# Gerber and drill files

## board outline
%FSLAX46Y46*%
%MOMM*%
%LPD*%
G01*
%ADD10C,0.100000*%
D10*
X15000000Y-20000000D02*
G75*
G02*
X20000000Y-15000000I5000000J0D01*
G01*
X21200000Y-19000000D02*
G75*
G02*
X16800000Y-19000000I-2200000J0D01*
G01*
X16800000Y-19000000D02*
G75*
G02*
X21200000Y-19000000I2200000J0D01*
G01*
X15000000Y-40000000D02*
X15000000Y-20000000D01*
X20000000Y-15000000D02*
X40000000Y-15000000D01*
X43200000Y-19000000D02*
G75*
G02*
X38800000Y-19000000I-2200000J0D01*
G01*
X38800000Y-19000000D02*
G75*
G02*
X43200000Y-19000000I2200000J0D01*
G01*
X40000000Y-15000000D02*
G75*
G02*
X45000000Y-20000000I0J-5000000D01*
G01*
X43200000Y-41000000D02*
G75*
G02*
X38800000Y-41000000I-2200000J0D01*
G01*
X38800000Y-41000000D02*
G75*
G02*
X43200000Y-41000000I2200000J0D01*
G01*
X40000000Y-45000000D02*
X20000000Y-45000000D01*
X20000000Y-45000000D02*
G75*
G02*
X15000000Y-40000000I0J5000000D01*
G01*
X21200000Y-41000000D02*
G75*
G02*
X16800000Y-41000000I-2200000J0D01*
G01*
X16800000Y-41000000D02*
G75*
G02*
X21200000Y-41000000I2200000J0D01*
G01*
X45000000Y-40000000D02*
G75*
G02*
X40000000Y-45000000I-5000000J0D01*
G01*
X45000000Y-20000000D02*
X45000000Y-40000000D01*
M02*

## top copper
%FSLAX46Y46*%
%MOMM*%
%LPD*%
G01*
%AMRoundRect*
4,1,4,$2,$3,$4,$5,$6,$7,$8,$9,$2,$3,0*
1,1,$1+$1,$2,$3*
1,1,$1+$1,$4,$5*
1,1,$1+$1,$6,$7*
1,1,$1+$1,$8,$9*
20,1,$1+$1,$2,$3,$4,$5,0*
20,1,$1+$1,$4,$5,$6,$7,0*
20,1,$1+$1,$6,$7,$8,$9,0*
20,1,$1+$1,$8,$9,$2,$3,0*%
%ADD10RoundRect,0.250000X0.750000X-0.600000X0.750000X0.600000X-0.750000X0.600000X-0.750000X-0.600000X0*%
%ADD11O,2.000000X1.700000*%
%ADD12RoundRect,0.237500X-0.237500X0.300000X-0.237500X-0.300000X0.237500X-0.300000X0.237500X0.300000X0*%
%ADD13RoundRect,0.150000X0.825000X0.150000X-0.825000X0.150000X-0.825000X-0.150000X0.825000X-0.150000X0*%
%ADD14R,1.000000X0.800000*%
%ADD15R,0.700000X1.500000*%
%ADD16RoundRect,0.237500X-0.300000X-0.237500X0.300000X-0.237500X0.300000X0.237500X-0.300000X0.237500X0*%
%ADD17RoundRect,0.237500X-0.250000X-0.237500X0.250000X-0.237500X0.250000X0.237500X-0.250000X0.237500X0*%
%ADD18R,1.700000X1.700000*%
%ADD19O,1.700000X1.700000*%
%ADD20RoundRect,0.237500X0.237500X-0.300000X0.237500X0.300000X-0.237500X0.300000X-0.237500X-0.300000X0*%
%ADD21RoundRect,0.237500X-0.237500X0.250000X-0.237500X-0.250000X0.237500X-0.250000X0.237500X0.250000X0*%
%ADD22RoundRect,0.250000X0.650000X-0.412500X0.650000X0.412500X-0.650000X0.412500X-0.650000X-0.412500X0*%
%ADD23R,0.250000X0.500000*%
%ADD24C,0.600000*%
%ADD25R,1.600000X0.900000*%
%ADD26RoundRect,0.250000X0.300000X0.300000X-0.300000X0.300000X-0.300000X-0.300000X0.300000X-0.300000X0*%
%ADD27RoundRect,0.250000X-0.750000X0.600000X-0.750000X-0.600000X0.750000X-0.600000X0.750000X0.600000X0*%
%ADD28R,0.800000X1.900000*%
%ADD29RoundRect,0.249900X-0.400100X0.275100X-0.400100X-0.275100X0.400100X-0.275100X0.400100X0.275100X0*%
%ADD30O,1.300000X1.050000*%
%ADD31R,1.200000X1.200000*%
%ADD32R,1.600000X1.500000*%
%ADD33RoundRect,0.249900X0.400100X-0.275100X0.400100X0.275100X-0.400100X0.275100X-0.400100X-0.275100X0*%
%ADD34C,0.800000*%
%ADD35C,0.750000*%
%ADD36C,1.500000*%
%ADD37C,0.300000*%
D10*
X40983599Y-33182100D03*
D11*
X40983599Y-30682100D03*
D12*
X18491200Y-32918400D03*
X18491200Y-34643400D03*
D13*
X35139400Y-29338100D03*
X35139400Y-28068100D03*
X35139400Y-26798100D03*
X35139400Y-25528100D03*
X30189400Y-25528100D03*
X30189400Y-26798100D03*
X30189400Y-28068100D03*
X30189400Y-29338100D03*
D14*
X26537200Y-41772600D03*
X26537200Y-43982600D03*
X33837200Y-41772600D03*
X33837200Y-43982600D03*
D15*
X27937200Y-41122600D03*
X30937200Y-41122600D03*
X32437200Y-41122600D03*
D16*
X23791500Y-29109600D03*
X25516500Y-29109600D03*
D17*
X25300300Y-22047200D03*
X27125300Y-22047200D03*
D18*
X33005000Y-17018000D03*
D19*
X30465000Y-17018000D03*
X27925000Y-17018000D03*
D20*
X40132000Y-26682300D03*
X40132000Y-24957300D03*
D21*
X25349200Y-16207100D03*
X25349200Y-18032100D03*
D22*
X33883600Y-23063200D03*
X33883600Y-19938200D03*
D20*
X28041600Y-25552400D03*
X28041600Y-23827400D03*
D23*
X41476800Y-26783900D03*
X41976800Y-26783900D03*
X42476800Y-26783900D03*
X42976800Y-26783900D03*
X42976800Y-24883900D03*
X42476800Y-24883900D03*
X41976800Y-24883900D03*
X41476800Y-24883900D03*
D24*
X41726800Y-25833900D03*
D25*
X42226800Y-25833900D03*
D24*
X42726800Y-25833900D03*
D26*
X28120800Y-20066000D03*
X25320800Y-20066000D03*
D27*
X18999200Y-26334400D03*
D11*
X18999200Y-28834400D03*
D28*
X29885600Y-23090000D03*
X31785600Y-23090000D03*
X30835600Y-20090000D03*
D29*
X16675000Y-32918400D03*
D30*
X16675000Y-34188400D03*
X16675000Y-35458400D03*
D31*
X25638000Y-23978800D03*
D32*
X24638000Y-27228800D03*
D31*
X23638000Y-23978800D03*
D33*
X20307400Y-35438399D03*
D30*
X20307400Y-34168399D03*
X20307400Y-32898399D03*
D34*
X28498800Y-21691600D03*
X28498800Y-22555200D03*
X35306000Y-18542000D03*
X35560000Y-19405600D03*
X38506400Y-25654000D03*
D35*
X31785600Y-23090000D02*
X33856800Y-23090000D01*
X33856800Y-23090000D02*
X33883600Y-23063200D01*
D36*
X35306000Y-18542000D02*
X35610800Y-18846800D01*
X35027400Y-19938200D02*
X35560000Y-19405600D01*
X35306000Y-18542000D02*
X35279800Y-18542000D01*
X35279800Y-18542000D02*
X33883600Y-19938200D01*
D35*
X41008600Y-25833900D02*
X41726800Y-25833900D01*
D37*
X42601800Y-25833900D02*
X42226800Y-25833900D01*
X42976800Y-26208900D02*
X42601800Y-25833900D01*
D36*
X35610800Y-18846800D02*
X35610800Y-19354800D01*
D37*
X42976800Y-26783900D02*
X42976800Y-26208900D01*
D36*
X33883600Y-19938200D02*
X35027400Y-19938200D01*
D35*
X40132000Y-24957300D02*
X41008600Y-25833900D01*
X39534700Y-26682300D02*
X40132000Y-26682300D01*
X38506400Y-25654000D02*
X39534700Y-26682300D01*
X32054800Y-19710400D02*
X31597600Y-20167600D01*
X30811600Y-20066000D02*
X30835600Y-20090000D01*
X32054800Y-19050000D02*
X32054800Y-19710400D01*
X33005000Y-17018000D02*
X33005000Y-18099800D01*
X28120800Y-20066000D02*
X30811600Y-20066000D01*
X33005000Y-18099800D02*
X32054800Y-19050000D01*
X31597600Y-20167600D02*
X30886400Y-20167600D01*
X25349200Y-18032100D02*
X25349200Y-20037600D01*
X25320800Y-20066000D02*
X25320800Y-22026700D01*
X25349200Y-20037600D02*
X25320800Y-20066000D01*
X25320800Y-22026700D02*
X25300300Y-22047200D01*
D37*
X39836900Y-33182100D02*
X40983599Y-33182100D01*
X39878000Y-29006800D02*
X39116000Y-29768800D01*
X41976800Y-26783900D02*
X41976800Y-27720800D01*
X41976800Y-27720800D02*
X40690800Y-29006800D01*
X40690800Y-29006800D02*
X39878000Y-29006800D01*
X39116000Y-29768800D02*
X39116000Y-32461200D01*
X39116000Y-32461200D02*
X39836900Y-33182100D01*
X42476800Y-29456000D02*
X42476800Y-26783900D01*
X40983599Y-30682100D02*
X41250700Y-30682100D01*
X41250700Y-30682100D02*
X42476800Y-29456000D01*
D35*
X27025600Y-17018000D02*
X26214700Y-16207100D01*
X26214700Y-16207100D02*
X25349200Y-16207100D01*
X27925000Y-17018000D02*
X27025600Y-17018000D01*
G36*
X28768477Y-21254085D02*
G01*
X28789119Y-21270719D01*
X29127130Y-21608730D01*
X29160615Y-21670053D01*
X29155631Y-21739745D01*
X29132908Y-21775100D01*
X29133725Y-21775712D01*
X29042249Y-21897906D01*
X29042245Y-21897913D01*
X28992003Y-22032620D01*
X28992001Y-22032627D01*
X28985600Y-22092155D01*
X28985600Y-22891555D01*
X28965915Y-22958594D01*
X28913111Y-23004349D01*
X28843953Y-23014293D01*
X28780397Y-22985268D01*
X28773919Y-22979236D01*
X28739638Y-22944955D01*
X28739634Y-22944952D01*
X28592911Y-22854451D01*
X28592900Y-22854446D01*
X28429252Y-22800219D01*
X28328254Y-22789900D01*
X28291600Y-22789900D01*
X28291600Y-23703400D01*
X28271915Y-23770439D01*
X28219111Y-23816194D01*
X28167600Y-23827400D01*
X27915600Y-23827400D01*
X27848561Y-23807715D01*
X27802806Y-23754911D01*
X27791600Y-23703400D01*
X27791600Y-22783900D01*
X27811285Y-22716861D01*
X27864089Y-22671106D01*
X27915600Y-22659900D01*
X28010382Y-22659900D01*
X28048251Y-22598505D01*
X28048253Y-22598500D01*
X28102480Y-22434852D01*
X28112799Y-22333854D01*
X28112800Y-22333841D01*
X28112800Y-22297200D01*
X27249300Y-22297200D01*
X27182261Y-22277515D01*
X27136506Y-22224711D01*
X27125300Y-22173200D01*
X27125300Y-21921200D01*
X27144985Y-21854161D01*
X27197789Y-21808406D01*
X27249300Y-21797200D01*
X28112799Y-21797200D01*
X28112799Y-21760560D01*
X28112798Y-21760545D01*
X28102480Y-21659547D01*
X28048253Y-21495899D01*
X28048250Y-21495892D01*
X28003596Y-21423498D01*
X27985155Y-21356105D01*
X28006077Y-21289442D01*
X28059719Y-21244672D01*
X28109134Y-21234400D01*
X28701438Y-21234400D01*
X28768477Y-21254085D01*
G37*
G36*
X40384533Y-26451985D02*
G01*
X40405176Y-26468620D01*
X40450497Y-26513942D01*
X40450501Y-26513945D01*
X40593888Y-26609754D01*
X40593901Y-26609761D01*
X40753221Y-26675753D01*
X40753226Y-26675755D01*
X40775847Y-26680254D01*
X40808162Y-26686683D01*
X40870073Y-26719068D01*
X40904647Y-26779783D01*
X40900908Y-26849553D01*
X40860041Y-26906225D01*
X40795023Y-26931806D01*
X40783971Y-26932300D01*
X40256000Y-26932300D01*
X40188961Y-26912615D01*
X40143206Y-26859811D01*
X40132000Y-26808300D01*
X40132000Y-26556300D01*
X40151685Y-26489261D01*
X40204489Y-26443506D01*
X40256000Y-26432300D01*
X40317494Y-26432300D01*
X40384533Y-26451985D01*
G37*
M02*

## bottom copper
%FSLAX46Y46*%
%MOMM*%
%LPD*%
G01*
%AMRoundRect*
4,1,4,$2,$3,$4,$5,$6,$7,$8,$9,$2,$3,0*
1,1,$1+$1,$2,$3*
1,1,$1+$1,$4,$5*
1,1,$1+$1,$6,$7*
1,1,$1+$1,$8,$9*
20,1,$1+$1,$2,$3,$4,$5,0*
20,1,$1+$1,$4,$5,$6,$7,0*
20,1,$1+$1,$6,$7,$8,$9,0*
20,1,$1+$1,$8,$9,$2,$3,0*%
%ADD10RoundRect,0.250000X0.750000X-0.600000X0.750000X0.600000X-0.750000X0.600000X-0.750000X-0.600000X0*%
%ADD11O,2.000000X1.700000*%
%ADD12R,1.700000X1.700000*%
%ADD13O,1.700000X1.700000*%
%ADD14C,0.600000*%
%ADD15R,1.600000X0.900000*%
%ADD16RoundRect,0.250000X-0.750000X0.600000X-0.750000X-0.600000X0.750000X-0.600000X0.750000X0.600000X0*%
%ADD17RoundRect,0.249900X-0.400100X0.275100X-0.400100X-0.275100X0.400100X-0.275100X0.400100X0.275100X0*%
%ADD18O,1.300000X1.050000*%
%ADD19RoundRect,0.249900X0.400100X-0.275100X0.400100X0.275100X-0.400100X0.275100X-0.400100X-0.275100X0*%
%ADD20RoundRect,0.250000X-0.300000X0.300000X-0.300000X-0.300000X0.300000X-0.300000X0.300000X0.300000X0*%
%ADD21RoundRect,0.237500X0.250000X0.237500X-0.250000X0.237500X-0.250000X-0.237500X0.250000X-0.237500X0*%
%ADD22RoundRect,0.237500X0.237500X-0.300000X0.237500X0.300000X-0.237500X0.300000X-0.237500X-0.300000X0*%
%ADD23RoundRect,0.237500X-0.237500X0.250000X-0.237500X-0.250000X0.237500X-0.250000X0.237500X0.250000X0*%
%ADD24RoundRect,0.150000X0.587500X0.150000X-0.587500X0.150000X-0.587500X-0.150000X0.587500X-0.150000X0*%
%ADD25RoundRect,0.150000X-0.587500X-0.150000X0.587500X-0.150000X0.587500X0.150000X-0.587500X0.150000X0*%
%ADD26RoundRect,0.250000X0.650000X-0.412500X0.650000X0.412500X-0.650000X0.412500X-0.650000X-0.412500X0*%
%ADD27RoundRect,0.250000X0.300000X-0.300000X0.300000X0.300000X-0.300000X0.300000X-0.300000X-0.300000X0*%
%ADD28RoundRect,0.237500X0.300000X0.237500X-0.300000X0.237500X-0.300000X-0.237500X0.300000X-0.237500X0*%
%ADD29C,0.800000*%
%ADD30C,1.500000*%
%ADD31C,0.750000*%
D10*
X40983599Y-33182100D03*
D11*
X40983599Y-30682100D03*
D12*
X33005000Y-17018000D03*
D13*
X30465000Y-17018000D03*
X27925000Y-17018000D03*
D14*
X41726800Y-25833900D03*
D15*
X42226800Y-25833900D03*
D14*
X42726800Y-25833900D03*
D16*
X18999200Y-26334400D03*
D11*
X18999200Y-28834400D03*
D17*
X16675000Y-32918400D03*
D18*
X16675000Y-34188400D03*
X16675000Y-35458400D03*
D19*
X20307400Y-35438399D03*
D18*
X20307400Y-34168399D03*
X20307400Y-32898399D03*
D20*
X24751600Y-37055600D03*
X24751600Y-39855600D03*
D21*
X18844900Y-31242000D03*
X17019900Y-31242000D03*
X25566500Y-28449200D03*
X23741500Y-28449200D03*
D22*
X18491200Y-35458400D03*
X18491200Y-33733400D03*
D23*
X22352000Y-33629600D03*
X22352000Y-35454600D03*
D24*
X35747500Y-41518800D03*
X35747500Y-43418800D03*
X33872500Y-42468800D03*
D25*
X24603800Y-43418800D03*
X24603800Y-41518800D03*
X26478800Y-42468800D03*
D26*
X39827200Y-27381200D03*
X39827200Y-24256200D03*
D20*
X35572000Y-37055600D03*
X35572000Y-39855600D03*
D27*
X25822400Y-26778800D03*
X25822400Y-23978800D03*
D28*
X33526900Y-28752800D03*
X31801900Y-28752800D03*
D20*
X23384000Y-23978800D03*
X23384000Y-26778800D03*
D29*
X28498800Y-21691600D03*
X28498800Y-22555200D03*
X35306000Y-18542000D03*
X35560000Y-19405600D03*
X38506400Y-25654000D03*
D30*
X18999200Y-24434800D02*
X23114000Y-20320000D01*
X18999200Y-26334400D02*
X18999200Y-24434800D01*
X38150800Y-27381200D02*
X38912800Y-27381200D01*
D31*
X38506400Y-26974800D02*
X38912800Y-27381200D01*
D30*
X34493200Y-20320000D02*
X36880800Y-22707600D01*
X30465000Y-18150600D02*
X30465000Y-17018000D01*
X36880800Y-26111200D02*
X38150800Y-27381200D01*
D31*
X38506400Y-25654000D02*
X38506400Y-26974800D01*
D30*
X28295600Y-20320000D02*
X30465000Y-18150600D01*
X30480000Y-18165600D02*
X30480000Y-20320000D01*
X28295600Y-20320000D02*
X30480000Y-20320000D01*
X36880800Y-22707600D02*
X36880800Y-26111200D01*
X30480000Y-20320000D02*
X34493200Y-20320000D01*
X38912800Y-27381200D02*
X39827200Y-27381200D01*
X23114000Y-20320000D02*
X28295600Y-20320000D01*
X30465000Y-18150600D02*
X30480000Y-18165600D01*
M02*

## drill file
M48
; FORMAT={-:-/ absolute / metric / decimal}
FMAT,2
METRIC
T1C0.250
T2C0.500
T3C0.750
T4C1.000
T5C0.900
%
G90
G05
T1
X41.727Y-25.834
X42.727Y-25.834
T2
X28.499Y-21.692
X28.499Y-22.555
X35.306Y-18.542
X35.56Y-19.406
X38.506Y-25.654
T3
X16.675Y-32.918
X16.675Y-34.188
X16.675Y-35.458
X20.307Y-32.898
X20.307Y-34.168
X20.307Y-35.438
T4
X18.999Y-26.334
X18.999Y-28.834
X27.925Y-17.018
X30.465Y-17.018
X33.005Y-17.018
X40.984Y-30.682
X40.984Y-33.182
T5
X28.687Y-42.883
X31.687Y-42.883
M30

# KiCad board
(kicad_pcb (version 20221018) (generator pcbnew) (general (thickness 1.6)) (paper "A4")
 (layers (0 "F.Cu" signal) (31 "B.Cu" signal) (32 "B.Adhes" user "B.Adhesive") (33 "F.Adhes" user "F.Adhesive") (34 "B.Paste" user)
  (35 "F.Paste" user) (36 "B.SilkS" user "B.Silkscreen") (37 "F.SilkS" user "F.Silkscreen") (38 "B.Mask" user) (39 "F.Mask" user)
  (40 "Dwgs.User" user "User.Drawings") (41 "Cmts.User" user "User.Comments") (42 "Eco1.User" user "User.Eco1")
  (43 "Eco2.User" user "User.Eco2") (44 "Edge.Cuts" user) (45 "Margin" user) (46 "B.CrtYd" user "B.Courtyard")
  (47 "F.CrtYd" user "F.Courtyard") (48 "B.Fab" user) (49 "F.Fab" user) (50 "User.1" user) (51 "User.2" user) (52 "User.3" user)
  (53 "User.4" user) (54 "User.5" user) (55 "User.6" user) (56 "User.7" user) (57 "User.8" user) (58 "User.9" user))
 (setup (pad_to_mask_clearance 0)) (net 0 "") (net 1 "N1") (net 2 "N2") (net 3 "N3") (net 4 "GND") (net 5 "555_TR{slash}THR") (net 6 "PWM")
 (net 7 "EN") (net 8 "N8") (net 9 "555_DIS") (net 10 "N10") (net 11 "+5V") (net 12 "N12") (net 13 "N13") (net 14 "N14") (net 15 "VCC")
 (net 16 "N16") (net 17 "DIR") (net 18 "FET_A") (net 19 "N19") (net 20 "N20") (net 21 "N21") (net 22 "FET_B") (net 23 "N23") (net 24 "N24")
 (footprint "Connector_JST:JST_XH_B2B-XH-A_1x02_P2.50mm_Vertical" (layer "F.Cu") (at 40.983599 33.1821 90)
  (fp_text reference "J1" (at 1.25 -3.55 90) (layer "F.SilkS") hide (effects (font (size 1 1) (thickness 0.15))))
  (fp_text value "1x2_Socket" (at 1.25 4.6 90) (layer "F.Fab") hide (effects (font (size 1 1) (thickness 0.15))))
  (pad "1" thru_hole roundrect (at 0 0 90) (size 1.7 2) (drill 1) (layers "*.Cu" "*.Mask") (roundrect_rratio 0.147059) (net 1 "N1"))
  (pad "2" thru_hole oval (at 2.5 0 90) (size 1.7 2) (drill 1) (layers "*.Cu" "*.Mask") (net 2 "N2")))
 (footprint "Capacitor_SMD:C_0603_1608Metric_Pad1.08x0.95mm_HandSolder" (layer "F.Cu") (at 18.4912 33.7809 -90)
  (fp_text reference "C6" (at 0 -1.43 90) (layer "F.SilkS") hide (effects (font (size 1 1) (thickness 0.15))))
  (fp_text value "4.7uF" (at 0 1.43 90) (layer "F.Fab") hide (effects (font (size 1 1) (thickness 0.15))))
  (pad "1" smd roundrect (at -0.8625 0 270) (size 1.075 0.95) (layers "F.Cu" "F.Paste" "F.Mask") (roundrect_rratio 0.25) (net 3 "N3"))
  (pad "2" smd roundrect (at 0.8625 0 270) (size 1.075 0.95) (layers "F.Cu" "F.Paste" "F.Mask") (roundrect_rratio 0.25) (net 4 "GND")))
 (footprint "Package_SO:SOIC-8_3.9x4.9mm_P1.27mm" (layer "F.Cu") (at 32.6644 27.4331 180)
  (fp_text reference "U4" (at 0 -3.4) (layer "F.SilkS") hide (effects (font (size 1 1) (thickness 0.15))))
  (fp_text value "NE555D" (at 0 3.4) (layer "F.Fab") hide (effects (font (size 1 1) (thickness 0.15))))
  (pad "1" smd roundrect (at -2.475 -1.905 180) (size 1.95 0.6) (layers "F.Cu" "F.Paste" "F.Mask") (roundrect_rratio 0.25) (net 4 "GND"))
  (pad "2" smd roundrect (at -2.475 -0.635 180) (size 1.95 0.6) (layers "F.Cu" "F.Paste" "F.Mask") (roundrect_rratio 0.25)
   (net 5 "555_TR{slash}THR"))
  (pad "3" smd roundrect (at -2.475 0.635 180) (size 1.95 0.6) (layers "F.Cu" "F.Paste" "F.Mask") (roundrect_rratio 0.25) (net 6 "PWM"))
  (pad "4" smd roundrect (at -2.475 1.905 180) (size 1.95 0.6) (layers "F.Cu" "F.Paste" "F.Mask") (roundrect_rratio 0.25) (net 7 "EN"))
  (pad "5" smd roundrect (at 2.475 1.905 180) (size 1.95 0.6) (layers "F.Cu" "F.Paste" "F.Mask") (roundrect_rratio 0.25) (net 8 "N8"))
  (pad "6" smd roundrect (at 2.475 0.635 180) (size 1.95 0.6) (layers "F.Cu" "F.Paste" "F.Mask") (roundrect_rratio 0.25)
   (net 5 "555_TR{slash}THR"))
  (pad "7" smd roundrect (at 2.475 -0.635 180) (size 1.95 0.6) (layers "F.Cu" "F.Paste" "F.Mask") (roundrect_rratio 0.25) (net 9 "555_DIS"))
  (pad "8" smd roundrect (at 2.475 -1.905 180) (size 1.95 0.6) (layers "F.Cu" "F.Paste" "F.Mask") (roundrect_rratio 0.25) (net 7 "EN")))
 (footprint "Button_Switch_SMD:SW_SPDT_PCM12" (layer "F.Cu") (at 30.1872 42.5526)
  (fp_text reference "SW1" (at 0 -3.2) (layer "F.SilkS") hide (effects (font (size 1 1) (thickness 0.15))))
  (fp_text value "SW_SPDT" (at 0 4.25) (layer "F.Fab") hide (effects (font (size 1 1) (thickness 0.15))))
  (pad "" smd rect (at -3.65 -0.78) (size 1 0.8) (layers "F.Cu" "F.Paste" "F.Mask"))
  (pad "" smd rect (at -3.65 1.43) (size 1 0.8) (layers "F.Cu" "F.Paste" "F.Mask"))
  (pad "" np_thru_hole circle (at -1.5 0.33) (size 0.9 0.9) (drill 0.9) (layers "*.Cu" "*.Mask"))
  (pad "" np_thru_hole circle (at 1.5 0.33) (size 0.9 0.9) (drill 0.9) (layers "*.Cu" "*.Mask"))
  (pad "" smd rect (at 3.65 -0.78) (size 1 0.8) (layers "F.Cu" "F.Paste" "F.Mask"))
  (pad "" smd rect (at 3.65 1.43) (size 1 0.8) (layers "F.Cu" "F.Paste" "F.Mask"))
  (pad "1" smd rect (at -2.25 -1.43) (size 0.7 1.5) (layers "F.Cu" "F.Paste" "F.Mask") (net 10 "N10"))
  (pad "2" smd rect (at 0.75 -1.43) (size 0.7 1.5) (layers "F.Cu" "F.Paste" "F.Mask") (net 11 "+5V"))
  (pad "3" smd rect (at 2.25 -1.43) (size 0.7 1.5) (layers "F.Cu" "F.Paste" "F.Mask") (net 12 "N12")))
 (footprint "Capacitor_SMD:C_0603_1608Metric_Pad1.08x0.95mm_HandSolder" (layer "F.Cu") (at 24.654 29.1096)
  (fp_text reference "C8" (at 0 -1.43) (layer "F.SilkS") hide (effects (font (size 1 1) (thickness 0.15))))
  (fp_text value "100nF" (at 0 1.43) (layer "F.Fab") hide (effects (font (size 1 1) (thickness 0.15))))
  (pad "1" smd roundrect (at -0.8625 0) (size 1.075 0.95) (layers "F.Cu" "F.Paste" "F.Mask") (roundrect_rratio 0.25)
   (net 5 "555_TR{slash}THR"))
  (pad "2" smd roundrect (at 0.8625 0) (size 1.075 0.95) (layers "F.Cu" "F.Paste" "F.Mask") (roundrect_rratio 0.25) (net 4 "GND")))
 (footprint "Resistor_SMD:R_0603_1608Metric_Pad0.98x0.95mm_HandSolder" (layer "F.Cu") (at 26.2128 22.0472)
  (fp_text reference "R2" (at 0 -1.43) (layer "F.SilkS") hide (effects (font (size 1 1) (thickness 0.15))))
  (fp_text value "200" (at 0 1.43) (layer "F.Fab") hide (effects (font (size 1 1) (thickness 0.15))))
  (pad "1" smd roundrect (at -0.9125 0) (size 0.975 0.95) (layers "F.Cu" "F.Paste" "F.Mask") (roundrect_rratio 0.25) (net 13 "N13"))
  (pad "2" smd roundrect (at 0.9125 0) (size 0.975 0.95) (layers "F.Cu" "F.Paste" "F.Mask") (roundrect_rratio 0.25) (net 4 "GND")))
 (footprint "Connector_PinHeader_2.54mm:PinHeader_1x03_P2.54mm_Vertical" (layer "F.Cu") (at 33.005 17.018 -90)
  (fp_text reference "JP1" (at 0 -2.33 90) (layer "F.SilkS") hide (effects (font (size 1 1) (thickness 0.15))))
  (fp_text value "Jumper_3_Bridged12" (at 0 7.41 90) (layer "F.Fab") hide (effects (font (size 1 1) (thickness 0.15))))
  (pad "1" thru_hole rect (at 0 0 270) (size 1.7 1.7) (drill 1) (layers "*.Cu" "*.Mask") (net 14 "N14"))
  (pad "2" thru_hole oval (at 0 2.54 270) (size 1.7 1.7) (drill 1) (layers "*.Cu" "*.Mask") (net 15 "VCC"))
  (pad "3" thru_hole oval (at 0 5.08 270) (size 1.7 1.7) (drill 1) (layers "*.Cu" "*.Mask") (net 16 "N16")))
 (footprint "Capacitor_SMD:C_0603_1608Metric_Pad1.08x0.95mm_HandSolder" (layer "F.Cu") (at 40.132 25.8198 90)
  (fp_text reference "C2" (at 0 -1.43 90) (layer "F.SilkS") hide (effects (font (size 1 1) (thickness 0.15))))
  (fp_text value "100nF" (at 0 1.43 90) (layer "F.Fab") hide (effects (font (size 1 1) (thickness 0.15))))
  (pad "1" smd roundrect (at -0.8625 0 90) (size 1.075 0.95) (layers "F.Cu" "F.Paste" "F.Mask") (roundrect_rratio 0.25) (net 15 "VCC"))
  (pad "2" smd roundrect (at 0.8625 0 90) (size 1.075 0.95) (layers "F.Cu" "F.Paste" "F.Mask") (roundrect_rratio 0.25) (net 4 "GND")))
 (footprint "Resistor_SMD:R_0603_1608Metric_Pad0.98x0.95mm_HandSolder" (layer "F.Cu") (at 25.3492 17.1196 -90)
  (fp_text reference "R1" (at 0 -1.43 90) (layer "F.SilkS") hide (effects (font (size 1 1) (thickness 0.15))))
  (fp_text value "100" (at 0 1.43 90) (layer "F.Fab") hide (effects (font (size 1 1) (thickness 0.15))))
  (pad "1" smd roundrect (at -0.9125 0 270) (size 0.975 0.95) (layers "F.Cu" "F.Paste" "F.Mask") (roundrect_rratio 0.25) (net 16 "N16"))
  (pad "2" smd roundrect (at 0.9125 0 270) (size 0.975 0.95) (layers "F.Cu" "F.Paste" "F.Mask") (roundrect_rratio 0.25) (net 13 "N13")))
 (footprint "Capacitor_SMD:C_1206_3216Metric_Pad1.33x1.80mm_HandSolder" (layer "F.Cu") (at 33.8836 21.5007 90)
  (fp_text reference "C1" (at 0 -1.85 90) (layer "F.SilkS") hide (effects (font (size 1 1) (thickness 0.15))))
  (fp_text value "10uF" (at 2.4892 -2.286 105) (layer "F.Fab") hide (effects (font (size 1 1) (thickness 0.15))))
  (pad "1" smd roundrect (at -1.5625 0 90) (size 1.325 1.8) (layers "F.Cu" "F.Paste" "F.Mask") (roundrect_rratio 0.188679) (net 11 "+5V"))
  (pad "2" smd roundrect (at 1.5625 0 90) (size 1.325 1.8) (layers "F.Cu" "F.Paste" "F.Mask") (roundrect_rratio 0.188679) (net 4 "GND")))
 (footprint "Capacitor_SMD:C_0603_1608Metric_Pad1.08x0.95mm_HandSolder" (layer "F.Cu") (at 28.0416 24.6899 90)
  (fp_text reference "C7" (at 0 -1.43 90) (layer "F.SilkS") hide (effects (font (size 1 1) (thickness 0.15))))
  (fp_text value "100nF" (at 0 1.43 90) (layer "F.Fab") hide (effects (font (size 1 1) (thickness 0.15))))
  (pad "1" smd roundrect (at -0.8625 0 90) (size 1.075 0.95) (layers "F.Cu" "F.Paste" "F.Mask") (roundrect_rratio 0.25) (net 8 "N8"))
  (pad "2" smd roundrect (at 0.8625 0 90) (size 1.075 0.95) (layers "F.Cu" "F.Paste" "F.Mask") (roundrect_rratio 0.25) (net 4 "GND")))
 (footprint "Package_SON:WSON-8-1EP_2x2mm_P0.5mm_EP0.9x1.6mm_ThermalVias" (layer "F.Cu") (at 42.2268 25.8339 90)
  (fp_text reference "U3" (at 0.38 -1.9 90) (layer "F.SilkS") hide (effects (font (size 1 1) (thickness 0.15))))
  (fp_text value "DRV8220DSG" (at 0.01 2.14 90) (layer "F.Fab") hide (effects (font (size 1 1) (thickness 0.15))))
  (pad "" smd rect (at 0 -0.4 90) (size 0.75 0.65) (layers "F.Paste"))
  (pad "" smd rect (at 0 0.4 90) (size 0.75 0.65) (layers "F.Paste"))
  (pad "1" smd rect (at -0.95 -0.75 90) (size 0.5 0.25) (layers "F.Cu" "F.Paste" "F.Mask") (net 15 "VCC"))
  (pad "2" smd rect (at -0.95 -0.25 90) (size 0.5 0.25) (layers "F.Cu" "F.Paste" "F.Mask") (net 1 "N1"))
  (pad "3" smd rect (at -0.95 0.25 90) (size 0.5 0.25) (layers "F.Cu" "F.Paste" "F.Mask") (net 2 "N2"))
  (pad "4" smd rect (at -0.95 0.75 90) (size 0.5 0.25) (layers "F.Cu" "F.Paste" "F.Mask") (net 4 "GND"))
  (pad "5" smd rect (at 0.95 0.75 90) (size 0.5 0.25) (layers "F.Cu" "F.Paste" "F.Mask") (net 6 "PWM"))
  (pad "6" smd rect (at 0.95 0.25 90) (size 0.5 0.25) (layers "F.Cu" "F.Paste" "F.Mask") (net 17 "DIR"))
  (pad "7" smd rect (at 0.95 -0.25 90) (size 0.5 0.25) (layers "F.Cu" "F.Paste" "F.Mask") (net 11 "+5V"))
  (pad "8" smd rect (at 0.95 -0.75 90) (size 0.5 0.25) (layers "F.Cu" "F.Paste" "F.Mask") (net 7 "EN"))
  (pad "9" thru_hole circle (at 0 -0.5 90) (size 0.6 0.6) (drill 0.25) (layers "*.Cu") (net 4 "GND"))
  (pad "9" smd rect (at 0 0 90) (size 0.9 1.6) (layers "F.Cu" "F.Mask") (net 4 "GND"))
  (pad "9" smd rect (at 0 0 90) (size 0.9 1.6) (layers "B.Cu") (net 4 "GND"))
  (pad "9" thru_hole circle (at 0 0.5 90) (size 0.6 0.6) (drill 0.25) (layers "*.Cu") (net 4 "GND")))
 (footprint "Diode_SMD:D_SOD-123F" (layer "F.Cu") (at 26.7208 20.066 180)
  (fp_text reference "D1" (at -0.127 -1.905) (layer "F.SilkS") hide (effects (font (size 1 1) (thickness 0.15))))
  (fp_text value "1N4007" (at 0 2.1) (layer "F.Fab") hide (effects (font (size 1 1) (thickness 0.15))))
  (pad "1" smd roundrect (at -1.4 0 180) (size 1.1 1.1) (layers "F.Cu" "F.Paste" "F.Mask") (roundrect_rratio 0.2272727273) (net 14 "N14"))
  (pad "2" smd roundrect (at 1.4 0 180) (size 1.1 1.1) (layers "F.Cu" "F.Paste" "F.Mask") (roundrect_rratio 0.2272727273) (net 13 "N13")))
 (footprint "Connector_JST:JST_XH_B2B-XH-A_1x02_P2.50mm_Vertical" (layer "F.Cu") (at 18.9992 26.3344 -90)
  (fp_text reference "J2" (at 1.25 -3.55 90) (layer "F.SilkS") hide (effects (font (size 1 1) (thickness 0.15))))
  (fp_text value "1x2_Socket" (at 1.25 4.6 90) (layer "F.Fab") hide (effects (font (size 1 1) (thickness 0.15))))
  (pad "1" thru_hole roundrect (at 0 0 270) (size 1.7 2) (drill 1) (layers "*.Cu" "*.Mask") (roundrect_rratio 0.147059) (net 15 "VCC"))
  (pad "2" thru_hole oval (at 2.5 0 270) (size 1.7 2) (drill 1) (layers "*.Cu" "*.Mask") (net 4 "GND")))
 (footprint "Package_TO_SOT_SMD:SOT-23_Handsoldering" (layer "F.Cu") (at 30.8356 21.59 90)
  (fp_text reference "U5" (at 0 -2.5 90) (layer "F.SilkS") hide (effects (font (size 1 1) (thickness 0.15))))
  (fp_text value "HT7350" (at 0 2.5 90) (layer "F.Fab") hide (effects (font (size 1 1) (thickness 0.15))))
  (pad "1" smd rect (at -1.5 -0.95 90) (size 1.9 0.8) (layers "F.Cu" "F.Paste" "F.Mask") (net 4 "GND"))
  (pad "2" smd rect (at -1.5 0.95 90) (size 1.9 0.8) (layers "F.Cu" "F.Paste" "F.Mask") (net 11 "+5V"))
  (pad "3" smd rect (at 1.5 0 90) (size 1.9 0.8) (layers "F.Cu" "F.Paste" "F.Mask") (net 14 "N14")))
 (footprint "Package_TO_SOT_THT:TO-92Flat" (layer "F.Cu") (at 16.675 32.9184 -90)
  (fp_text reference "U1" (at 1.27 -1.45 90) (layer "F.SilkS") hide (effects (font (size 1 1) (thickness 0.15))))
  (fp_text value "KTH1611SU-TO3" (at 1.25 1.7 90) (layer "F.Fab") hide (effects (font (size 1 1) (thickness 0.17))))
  (pad "1" thru_hole roundrect (at 0 0 270) (size 1.05 1.3) (drill 0.75) (layers "*.Cu" "*.Mask") (roundrect_rratio 0.238) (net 3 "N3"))
  (pad "2" thru_hole oval (at 1.27 0 270) (size 1.05 1.3) (drill 0.75) (layers "*.Cu" "*.Mask") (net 4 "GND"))
  (pad "3" thru_hole oval (at 2.54 0 270) (size 1.05 1.3) (drill 0.75) (layers "*.Cu" "*.Mask") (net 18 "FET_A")))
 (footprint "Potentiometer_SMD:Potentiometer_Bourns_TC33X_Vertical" (layer "F.Cu") (at 24.638 25.7788 -90)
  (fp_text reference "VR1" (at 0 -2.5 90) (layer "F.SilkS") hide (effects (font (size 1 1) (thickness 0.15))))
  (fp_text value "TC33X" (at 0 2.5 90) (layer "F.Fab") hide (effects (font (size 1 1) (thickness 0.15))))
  (pad "1" smd rect (at -1.8 -1 270) (size 1.2 1.2) (layers "F.Cu" "F.Paste" "F.Mask") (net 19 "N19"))
  (pad "2" smd rect (at 1.45 0 270) (size 1.5 1.6) (layers "F.Cu" "F.Paste" "F.Mask") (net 5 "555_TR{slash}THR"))
  (pad "3" smd rect (at -1.8 1 270) (size 1.2 1.2) (layers "F.Cu" "F.Paste" "F.Mask") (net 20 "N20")))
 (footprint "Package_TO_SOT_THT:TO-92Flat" (layer "F.Cu") (at 20.3074 35.438399 90)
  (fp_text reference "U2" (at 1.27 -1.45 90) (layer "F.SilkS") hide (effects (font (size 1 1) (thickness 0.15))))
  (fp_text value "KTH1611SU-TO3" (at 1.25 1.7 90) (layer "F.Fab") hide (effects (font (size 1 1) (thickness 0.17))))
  (pad "1" thru_hole roundrect (at 0 0 90) (size 1.05 1.3) (drill 0.75) (layers "*.Cu" "*.Mask") (roundrect_rratio 0.238) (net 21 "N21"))
  (pad "2" thru_hole oval (at 1.27 0 90) (size 1.05 1.3) (drill 0.75) (layers "*.Cu" "*.Mask") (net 4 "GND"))
  (pad "3" thru_hole oval (at 2.54 0 90) (size 1.05 1.3) (drill 0.75) (layers "*.Cu" "*.Mask") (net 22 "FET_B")))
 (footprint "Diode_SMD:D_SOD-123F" (layer "B.Cu") (at 24.7516 38.4556 -90)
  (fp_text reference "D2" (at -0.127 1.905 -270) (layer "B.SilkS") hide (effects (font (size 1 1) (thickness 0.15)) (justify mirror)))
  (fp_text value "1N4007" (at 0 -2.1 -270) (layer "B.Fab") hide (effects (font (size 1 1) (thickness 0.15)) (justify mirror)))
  (pad "1" smd roundrect (at -1.4 0 270) (size 1.1 1.1) (layers "B.Cu" "B.Paste" "B.Mask") (roundrect_rratio 0.2272727273) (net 7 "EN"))
  (pad "2" smd roundrect (at 1.4 0 270) (size 1.1 1.1) (layers "B.Cu" "B.Paste" "B.Mask") (roundrect_rratio 0.2272727273) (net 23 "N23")))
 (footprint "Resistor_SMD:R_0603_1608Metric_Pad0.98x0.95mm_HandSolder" (layer "B.Cu") (at 17.9324 31.242 180)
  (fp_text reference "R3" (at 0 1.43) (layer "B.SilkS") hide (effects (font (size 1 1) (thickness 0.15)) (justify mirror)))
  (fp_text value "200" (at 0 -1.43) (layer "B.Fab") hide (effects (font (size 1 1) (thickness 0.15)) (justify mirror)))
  (pad "1" smd roundrect (at -0.9125 0 180) (size 0.975 0.95) (layers "B.Cu" "B.Paste" "B.Mask") (roundrect_rratio 0.25) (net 11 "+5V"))
  (pad "2" smd roundrect (at 0.9125 0 180) (size 0.975 0.95) (layers "B.Cu" "B.Paste" "B.Mask") (roundrect_rratio 0.25) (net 3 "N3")))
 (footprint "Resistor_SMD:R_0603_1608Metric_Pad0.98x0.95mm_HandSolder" (layer "B.Cu") (at 24.654 28.4492 180)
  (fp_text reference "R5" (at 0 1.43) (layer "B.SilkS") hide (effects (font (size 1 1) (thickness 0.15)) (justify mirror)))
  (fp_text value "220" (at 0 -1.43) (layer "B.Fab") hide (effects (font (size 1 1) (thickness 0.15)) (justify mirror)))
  (pad "1" smd roundrect (at -0.9125 0 180) (size 0.975 0.95) (layers "B.Cu" "B.Paste" "B.Mask") (roundrect_rratio 0.25) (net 7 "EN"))
  (pad "2" smd roundrect (at 0.9125 0 180) (size 0.975 0.95) (layers "B.Cu" "B.Paste" "B.Mask") (roundrect_rratio 0.25) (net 9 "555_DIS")))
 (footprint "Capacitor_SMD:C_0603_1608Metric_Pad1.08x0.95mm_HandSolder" (layer "B.Cu") (at 18.4912 34.5959 90)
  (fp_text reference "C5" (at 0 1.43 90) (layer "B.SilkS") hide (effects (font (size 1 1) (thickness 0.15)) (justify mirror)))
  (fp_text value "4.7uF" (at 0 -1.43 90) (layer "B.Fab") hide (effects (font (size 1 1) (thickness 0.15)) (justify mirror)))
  (pad "1" smd roundrect (at -0.8625 0 90) (size 1.075 0.95) (layers "B.Cu" "B.Paste" "B.Mask") (roundrect_rratio 0.25) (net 21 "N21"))
  (pad "2" smd roundrect (at 0.8625 0 90) (size 1.075 0.95) (layers "B.Cu" "B.Paste" "B.Mask") (roundrect_rratio 0.25) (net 4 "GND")))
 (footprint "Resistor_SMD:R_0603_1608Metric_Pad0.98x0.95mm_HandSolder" (layer "B.Cu") (at 22.352 34.5421 -90)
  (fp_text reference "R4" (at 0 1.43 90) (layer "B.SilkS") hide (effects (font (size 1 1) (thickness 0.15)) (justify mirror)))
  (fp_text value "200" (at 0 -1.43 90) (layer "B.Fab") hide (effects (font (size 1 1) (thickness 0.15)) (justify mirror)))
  (pad "1" smd roundrect (at -0.9125 0 270) (size 0.975 0.95) (layers "B.Cu" "B.Paste" "B.Mask") (roundrect_rratio 0.25) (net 11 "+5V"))
  (pad "2" smd roundrect (at 0.9125 0 270) (size 0.975 0.95) (layers "B.Cu" "B.Paste" "B.Mask") (roundrect_rratio 0.25) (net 21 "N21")))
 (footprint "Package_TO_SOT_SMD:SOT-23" (layer "B.Cu") (at 34.81 42.4688 180)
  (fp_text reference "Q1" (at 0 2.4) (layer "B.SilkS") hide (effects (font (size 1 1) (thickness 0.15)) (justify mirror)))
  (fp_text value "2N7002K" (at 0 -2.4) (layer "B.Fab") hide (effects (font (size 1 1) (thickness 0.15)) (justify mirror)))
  (pad "1" smd roundrect (at -0.9375 0.95 180) (size 1.475 0.6) (layers "B.Cu" "B.Paste" "B.Mask") (roundrect_rratio 0.25) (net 18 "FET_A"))
  (pad "2" smd roundrect (at -0.9375 -0.95 180) (size 1.475 0.6) (layers "B.Cu" "B.Paste" "B.Mask") (roundrect_rratio 0.25) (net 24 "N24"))
  (pad "3" smd roundrect (at 0.9375 0 180) (size 1.475 0.6) (layers "B.Cu" "B.Paste" "B.Mask") (roundrect_rratio 0.25) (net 12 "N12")))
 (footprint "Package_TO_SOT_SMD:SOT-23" (layer "B.Cu") (at 25.5413 42.4688)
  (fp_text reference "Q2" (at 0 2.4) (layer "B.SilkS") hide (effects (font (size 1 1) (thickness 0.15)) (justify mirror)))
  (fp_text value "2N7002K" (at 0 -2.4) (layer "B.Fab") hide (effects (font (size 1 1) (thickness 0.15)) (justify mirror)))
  (pad "1" smd roundrect (at -0.9375 0.95) (size 1.475 0.6) (layers "B.Cu" "B.Paste" "B.Mask") (roundrect_rratio 0.25) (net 22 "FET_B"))
  (pad "2" smd roundrect (at -0.9375 -0.95) (size 1.475 0.6) (layers "B.Cu" "B.Paste" "B.Mask") (roundrect_rratio 0.25) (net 23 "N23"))
  (pad "3" smd roundrect (at 0.9375 0) (size 1.475 0.6) (layers "B.Cu" "B.Paste" "B.Mask") (roundrect_rratio 0.25) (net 10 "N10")))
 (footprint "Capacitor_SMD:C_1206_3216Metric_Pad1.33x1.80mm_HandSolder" (layer "B.Cu") (at 39.8272 25.8187 90)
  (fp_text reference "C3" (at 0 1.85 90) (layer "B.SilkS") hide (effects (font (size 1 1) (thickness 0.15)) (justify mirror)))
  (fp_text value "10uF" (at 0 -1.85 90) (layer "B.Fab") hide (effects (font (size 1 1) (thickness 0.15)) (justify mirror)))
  (pad "1" smd roundrect (at -1.5625 0 90) (size 1.325 1.8) (layers "B.Cu" "B.Paste" "B.Mask") (roundrect_rratio 0.188679) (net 15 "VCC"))
  (pad "2" smd roundrect (at 1.5625 0 90) (size 1.325 1.8) (layers "B.Cu" "B.Paste" "B.Mask") (roundrect_rratio 0.188679) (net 4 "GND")))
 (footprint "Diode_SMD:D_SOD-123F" (layer "B.Cu") (at 35.572 38.4556 -90)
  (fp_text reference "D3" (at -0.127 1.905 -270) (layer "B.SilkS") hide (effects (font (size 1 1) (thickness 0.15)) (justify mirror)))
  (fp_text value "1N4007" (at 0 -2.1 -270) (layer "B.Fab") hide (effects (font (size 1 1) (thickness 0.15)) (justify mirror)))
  (pad "1" smd roundrect (at -1.4 0 270) (size 1.1 1.1) (layers "B.Cu" "B.Paste" "B.Mask") (roundrect_rratio 0.2272727273) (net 7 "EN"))
  (pad "2" smd roundrect (at 1.4 0 270) (size 1.1 1.1) (layers "B.Cu" "B.Paste" "B.Mask") (roundrect_rratio 0.2272727273) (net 24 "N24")))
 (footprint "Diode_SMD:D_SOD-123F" (layer "B.Cu") (at 25.8224 25.3788 90)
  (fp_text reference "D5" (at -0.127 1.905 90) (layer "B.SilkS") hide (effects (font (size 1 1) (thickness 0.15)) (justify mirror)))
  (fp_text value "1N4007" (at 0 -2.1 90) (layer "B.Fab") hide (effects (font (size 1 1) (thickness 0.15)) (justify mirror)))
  (pad "1" smd roundrect (at -1.4 0 90) (size 1.1 1.1) (layers "B.Cu" "B.Paste" "B.Mask") (roundrect_rratio 0.2272727273) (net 9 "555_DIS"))
  (pad "2" smd roundrect (at 1.4 0 90) (size 1.1 1.1) (layers "B.Cu" "B.Paste" "B.Mask") (roundrect_rratio 0.2272727273) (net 19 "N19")))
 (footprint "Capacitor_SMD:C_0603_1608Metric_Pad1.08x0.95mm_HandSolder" (layer "B.Cu") (at 32.6644 28.7528 180)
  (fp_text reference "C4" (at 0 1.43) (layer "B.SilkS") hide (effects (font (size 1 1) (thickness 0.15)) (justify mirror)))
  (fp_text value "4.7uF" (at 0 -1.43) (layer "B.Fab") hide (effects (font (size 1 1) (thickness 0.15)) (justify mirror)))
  (pad "1" smd roundrect (at -0.8625 0 180) (size 1.075 0.95) (layers "B.Cu" "B.Paste" "B.Mask") (roundrect_rratio 0.25) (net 4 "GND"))
  (pad "2" smd roundrect (at 0.8625 0 180) (size 1.075 0.95) (layers "B.Cu" "B.Paste" "B.Mask") (roundrect_rratio 0.25) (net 7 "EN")))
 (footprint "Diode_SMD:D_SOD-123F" (layer "B.Cu") (at 23.384 25.3788 -90)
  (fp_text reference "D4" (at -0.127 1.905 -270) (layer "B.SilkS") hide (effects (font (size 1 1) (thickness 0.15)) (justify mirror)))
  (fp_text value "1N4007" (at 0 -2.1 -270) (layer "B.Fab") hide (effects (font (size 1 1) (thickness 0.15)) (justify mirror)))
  (pad "1" smd roundrect (at -1.4 0 270) (size 1.1 1.1) (layers "B.Cu" "B.Paste" "B.Mask") (roundrect_rratio 0.2272727273) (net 20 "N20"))
  (pad "2" smd roundrect (at 1.4 0 270) (size 1.1 1.1) (layers "B.Cu" "B.Paste" "B.Mask") (roundrect_rratio 0.2272727273) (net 9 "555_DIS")))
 (gr_arc (start 15 20) (mid 16.464466 16.464466) (end 20 15) (stroke (width 0.1) (type default)) (layer "Edge.Cuts"))
 (gr_circle (center 19 19) (end 21.2 19) (stroke (width 0.1) (type default)) (fill none) (layer "Edge.Cuts"))
 (gr_line (start 15 40) (end 15 20) (stroke (width 0.1) (type default)) (layer "Edge.Cuts"))
 (gr_line (start 20 15) (end 40 15) (stroke (width 0.1) (type default)) (layer "Edge.Cuts"))
 (gr_circle (center 41 19) (end 43.2 19) (stroke (width 0.1) (type default)) (fill none) (layer "Edge.Cuts"))
 (gr_arc (start 40 15) (mid 43.535534 16.464466) (end 45 20) (stroke (width 0.1) (type default)) (layer "Edge.Cuts"))
 (gr_circle (center 41 41) (end 43.2 41) (stroke (width 0.1) (type default)) (fill none) (layer "Edge.Cuts"))
 (gr_line (start 40 45) (end 20 45) (stroke (width 0.1) (type default)) (layer "Edge.Cuts"))
 (gr_arc (start 20 45) (mid 16.464466 43.535534) (end 15 40) (stroke (width 0.1) (type default)) (layer "Edge.Cuts"))
 (gr_circle (center 19 41) (end 21.2 41) (stroke (width 0.1) (type default)) (fill none) (layer "Edge.Cuts"))
 (gr_arc (start 45 40) (mid 43.535534 43.535534) (end 40 45) (stroke (width 0.1) (type default)) (layer "Edge.Cuts"))
 (gr_line (start 45 20) (end 45 40) (stroke (width 0.1) (type default)) (layer "Edge.Cuts"))
 (segment (start 31.7856 23.09) (end 33.8568 23.09) (width 0.75) (layer "F.Cu") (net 11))
 (segment (start 33.8568 23.09) (end 33.8836 23.0632) (width 0.75) (layer "F.Cu") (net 11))
 (segment (start 35.306 18.542) (end 35.6108 18.8468) (width 1.5) (layer "F.Cu") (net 4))
 (segment (start 35.0274 19.9382) (end 35.56 19.4056) (width 1.5) (layer "F.Cu") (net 4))
 (segment (start 35.306 18.542) (end 35.2798 18.542) (width 1.5) (layer "F.Cu") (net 4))
 (segment (start 35.2798 18.542) (end 33.8836 19.9382) (width 1.5) (layer "F.Cu") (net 4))
 (segment (start 41.0086 25.8339) (end 41.7268 25.8339) (width 0.75) (layer "F.Cu") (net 4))
 (segment (start 42.6018 25.8339) (end 42.2268 25.8339) (width 0.3) (layer "F.Cu") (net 4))
 (segment (start 42.9768 26.2089) (end 42.6018 25.8339) (width 0.3) (layer "F.Cu") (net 4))
 (segment (start 35.6108 18.8468) (end 35.6108 19.3548) (width 1.5) (layer "F.Cu") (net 4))
 (segment (start 42.9768 26.7839) (end 42.9768 26.2089) (width 0.3) (layer "F.Cu") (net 4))
 (segment (start 33.8836 19.9382) (end 35.0274 19.9382) (width 1.5) (layer "F.Cu") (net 4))
 (segment (start 40.132 24.9573) (end 41.0086 25.8339) (width 0.75) (layer "F.Cu") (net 4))
 (via (at 28.4988 21.6916) (size 0.8) (drill 0.5) (layers "F.Cu" "B.Cu") (free) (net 4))
 (via (at 28.4988 22.5552) (size 0.8) (drill 0.5) (layers "F.Cu" "B.Cu") (free) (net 4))
 (via (at 35.306 18.542) (size 0.8) (drill 0.5) (layers "F.Cu" "B.Cu") (free) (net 4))
 (via (at 35.56 19.4056) (size 0.8) (drill 0.5) (layers "F.Cu" "B.Cu") (free) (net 4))
 (segment (start 39.5347 26.6823) (end 40.132 26.6823) (width 0.75) (layer "F.Cu") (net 15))
 (segment (start 38.5064 25.654) (end 39.5347 26.6823) (width 0.75) (layer "F.Cu") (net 15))
 (via (at 38.5064 25.654) (size 0.8) (drill 0.5) (layers "F.Cu" "B.Cu") (free) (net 15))
 (segment (start 18.9992 24.4348) (end 23.114 20.32) (width 1.5) (layer "B.Cu") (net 15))
 (segment (start 18.9992 26.3344) (end 18.9992 24.4348) (width 1.5) (layer "B.Cu") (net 15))
 (segment (start 38.1508 27.3812) (end 38.9128 27.3812) (width 1.5) (layer "B.Cu") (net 15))
 (segment (start 38.5064 26.9748) (end 38.9128 27.3812) (width 0.75) (layer "B.Cu") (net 15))
 (segment (start 34.4932 20.32) (end 36.8808 22.7076) (width 1.5) (layer "B.Cu") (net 15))
 (segment (start 30.465 18.1506) (end 30.465 17.018) (width 1.5) (layer "B.Cu") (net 15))
 (segment (start 36.8808 26.1112) (end 38.1508 27.3812) (width 1.5) (layer "B.Cu") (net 15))
 (segment (start 38.5064 25.654) (end 38.5064 26.9748) (width 0.75) (layer "B.Cu") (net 15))
 (segment (start 28.2956 20.32) (end 30.465 18.1506) (width 1.5) (layer "B.Cu") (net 15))
 (segment (start 30.48 18.1656) (end 30.48 20.32) (width 1.5) (layer "B.Cu") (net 15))
 (segment (start 28.2956 20.32) (end 30.48 20.32) (width 1.5) (layer "B.Cu") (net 15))
 (segment (start 36.8808 22.7076) (end 36.8808 26.1112) (width 1.5) (layer "B.Cu") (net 15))
 (segment (start 30.48 20.32) (end 34.4932 20.32) (width 1.5) (layer "B.Cu") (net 15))
 (segment (start 38.9128 27.3812) (end 39.8272 27.3812) (width 1.5) (layer "B.Cu") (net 15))
 (segment (start 23.114 20.32) (end 28.2956 20.32) (width 1.5) (layer "B.Cu") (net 15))
 (segment (start 30.465 18.1506) (end 30.48 18.1656) (width 1.5) (layer "B.Cu") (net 15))
 (segment (start 32.0548 19.7104) (end 31.5976 20.1676) (width 0.75) (layer "F.Cu") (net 14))
 (segment (start 30.8116 20.066) (end 30.8356 20.09) (width 0.75) (layer "F.Cu") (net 14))
 (segment (start 32.0548 19.05) (end 32.0548 19.7104) (width 0.75) (layer "F.Cu") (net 14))
 (segment (start 33.005 17.018) (end 33.005 18.0998) (width 0.75) (layer "F.Cu") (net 14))
 (segment (start 28.1208 20.066) (end 30.8116 20.066) (width 0.75) (layer "F.Cu") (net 14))
 (segment (start 33.005 18.0998) (end 32.0548 19.05) (width 0.75) (layer "F.Cu") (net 14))
 (segment (start 31.5976 20.1676) (end 30.8864 20.1676) (width 0.75) (layer "F.Cu") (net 14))
 (segment (start 25.3492 18.0321) (end 25.3492 20.0376) (width 0.75) (layer "F.Cu") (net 13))
 (segment (start 25.3208 20.066) (end 25.3208 22.0267) (width 0.75) (layer "F.Cu") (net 13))
 (segment (start 25.3492 20.0376) (end 25.3208 20.066) (width 0.75) (layer "F.Cu") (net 13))
 (segment (start 25.3208 22.0267) (end 25.3003 22.0472) (width 0.75) (layer "F.Cu") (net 13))
 (segment (start 39.8369 33.1821) (end 40.983599 33.1821) (width 0.3) (layer "F.Cu") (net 1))
 (segment (start 39.878 29.0068) (end 39.116 29.7688) (width 0.3) (layer "F.Cu") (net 1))
 (segment (start 41.9768 26.7839) (end 41.9768 27.7208) (width 0.3) (layer "F.Cu") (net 1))
 (segment (start 41.9768 27.7208) (end 40.6908 29.0068) (width 0.3) (layer "F.Cu") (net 1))
 (segment (start 40.6908 29.0068) (end 39.878 29.0068) (width 0.3) (layer "F.Cu") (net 1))
 (segment (start 39.116 29.7688) (end 39.116 32.4612) (width 0.3) (layer "F.Cu") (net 1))
 (segment (start 39.116 32.4612) (end 39.8369 33.1821) (width 0.3) (layer "F.Cu") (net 1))
 (segment (start 42.4768 29.456) (end 42.4768 26.7839) (width 0.3) (layer "F.Cu") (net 2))
 (segment (start 40.983599 30.6821) (end 41.2507 30.6821) (width 0.3) (layer "F.Cu") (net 2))
 (segment (start 41.2507 30.6821) (end 42.4768 29.456) (width 0.3) (layer "F.Cu") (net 2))
 (segment (start 27.0256 17.018) (end 26.2147 16.2071) (width 0.75) (layer "F.Cu") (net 16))
 (segment (start 26.2147 16.2071) (end 25.3492 16.2071) (width 0.75) (layer "F.Cu") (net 16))
 (segment (start 27.925 17.018) (end 27.0256 17.018) (width 0.75) (layer "F.Cu") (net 16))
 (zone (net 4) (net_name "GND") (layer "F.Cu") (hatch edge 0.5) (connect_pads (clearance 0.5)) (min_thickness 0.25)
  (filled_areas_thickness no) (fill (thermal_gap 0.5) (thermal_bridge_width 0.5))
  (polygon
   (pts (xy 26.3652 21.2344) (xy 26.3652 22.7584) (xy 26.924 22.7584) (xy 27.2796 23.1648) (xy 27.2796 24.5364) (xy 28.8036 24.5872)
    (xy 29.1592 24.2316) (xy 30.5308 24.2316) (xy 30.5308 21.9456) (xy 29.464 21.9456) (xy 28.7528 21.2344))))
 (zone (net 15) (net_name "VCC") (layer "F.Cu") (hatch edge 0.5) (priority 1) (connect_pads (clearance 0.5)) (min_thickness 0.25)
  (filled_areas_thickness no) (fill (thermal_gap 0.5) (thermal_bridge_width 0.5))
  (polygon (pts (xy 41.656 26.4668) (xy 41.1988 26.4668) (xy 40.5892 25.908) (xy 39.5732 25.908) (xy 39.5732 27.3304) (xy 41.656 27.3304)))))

